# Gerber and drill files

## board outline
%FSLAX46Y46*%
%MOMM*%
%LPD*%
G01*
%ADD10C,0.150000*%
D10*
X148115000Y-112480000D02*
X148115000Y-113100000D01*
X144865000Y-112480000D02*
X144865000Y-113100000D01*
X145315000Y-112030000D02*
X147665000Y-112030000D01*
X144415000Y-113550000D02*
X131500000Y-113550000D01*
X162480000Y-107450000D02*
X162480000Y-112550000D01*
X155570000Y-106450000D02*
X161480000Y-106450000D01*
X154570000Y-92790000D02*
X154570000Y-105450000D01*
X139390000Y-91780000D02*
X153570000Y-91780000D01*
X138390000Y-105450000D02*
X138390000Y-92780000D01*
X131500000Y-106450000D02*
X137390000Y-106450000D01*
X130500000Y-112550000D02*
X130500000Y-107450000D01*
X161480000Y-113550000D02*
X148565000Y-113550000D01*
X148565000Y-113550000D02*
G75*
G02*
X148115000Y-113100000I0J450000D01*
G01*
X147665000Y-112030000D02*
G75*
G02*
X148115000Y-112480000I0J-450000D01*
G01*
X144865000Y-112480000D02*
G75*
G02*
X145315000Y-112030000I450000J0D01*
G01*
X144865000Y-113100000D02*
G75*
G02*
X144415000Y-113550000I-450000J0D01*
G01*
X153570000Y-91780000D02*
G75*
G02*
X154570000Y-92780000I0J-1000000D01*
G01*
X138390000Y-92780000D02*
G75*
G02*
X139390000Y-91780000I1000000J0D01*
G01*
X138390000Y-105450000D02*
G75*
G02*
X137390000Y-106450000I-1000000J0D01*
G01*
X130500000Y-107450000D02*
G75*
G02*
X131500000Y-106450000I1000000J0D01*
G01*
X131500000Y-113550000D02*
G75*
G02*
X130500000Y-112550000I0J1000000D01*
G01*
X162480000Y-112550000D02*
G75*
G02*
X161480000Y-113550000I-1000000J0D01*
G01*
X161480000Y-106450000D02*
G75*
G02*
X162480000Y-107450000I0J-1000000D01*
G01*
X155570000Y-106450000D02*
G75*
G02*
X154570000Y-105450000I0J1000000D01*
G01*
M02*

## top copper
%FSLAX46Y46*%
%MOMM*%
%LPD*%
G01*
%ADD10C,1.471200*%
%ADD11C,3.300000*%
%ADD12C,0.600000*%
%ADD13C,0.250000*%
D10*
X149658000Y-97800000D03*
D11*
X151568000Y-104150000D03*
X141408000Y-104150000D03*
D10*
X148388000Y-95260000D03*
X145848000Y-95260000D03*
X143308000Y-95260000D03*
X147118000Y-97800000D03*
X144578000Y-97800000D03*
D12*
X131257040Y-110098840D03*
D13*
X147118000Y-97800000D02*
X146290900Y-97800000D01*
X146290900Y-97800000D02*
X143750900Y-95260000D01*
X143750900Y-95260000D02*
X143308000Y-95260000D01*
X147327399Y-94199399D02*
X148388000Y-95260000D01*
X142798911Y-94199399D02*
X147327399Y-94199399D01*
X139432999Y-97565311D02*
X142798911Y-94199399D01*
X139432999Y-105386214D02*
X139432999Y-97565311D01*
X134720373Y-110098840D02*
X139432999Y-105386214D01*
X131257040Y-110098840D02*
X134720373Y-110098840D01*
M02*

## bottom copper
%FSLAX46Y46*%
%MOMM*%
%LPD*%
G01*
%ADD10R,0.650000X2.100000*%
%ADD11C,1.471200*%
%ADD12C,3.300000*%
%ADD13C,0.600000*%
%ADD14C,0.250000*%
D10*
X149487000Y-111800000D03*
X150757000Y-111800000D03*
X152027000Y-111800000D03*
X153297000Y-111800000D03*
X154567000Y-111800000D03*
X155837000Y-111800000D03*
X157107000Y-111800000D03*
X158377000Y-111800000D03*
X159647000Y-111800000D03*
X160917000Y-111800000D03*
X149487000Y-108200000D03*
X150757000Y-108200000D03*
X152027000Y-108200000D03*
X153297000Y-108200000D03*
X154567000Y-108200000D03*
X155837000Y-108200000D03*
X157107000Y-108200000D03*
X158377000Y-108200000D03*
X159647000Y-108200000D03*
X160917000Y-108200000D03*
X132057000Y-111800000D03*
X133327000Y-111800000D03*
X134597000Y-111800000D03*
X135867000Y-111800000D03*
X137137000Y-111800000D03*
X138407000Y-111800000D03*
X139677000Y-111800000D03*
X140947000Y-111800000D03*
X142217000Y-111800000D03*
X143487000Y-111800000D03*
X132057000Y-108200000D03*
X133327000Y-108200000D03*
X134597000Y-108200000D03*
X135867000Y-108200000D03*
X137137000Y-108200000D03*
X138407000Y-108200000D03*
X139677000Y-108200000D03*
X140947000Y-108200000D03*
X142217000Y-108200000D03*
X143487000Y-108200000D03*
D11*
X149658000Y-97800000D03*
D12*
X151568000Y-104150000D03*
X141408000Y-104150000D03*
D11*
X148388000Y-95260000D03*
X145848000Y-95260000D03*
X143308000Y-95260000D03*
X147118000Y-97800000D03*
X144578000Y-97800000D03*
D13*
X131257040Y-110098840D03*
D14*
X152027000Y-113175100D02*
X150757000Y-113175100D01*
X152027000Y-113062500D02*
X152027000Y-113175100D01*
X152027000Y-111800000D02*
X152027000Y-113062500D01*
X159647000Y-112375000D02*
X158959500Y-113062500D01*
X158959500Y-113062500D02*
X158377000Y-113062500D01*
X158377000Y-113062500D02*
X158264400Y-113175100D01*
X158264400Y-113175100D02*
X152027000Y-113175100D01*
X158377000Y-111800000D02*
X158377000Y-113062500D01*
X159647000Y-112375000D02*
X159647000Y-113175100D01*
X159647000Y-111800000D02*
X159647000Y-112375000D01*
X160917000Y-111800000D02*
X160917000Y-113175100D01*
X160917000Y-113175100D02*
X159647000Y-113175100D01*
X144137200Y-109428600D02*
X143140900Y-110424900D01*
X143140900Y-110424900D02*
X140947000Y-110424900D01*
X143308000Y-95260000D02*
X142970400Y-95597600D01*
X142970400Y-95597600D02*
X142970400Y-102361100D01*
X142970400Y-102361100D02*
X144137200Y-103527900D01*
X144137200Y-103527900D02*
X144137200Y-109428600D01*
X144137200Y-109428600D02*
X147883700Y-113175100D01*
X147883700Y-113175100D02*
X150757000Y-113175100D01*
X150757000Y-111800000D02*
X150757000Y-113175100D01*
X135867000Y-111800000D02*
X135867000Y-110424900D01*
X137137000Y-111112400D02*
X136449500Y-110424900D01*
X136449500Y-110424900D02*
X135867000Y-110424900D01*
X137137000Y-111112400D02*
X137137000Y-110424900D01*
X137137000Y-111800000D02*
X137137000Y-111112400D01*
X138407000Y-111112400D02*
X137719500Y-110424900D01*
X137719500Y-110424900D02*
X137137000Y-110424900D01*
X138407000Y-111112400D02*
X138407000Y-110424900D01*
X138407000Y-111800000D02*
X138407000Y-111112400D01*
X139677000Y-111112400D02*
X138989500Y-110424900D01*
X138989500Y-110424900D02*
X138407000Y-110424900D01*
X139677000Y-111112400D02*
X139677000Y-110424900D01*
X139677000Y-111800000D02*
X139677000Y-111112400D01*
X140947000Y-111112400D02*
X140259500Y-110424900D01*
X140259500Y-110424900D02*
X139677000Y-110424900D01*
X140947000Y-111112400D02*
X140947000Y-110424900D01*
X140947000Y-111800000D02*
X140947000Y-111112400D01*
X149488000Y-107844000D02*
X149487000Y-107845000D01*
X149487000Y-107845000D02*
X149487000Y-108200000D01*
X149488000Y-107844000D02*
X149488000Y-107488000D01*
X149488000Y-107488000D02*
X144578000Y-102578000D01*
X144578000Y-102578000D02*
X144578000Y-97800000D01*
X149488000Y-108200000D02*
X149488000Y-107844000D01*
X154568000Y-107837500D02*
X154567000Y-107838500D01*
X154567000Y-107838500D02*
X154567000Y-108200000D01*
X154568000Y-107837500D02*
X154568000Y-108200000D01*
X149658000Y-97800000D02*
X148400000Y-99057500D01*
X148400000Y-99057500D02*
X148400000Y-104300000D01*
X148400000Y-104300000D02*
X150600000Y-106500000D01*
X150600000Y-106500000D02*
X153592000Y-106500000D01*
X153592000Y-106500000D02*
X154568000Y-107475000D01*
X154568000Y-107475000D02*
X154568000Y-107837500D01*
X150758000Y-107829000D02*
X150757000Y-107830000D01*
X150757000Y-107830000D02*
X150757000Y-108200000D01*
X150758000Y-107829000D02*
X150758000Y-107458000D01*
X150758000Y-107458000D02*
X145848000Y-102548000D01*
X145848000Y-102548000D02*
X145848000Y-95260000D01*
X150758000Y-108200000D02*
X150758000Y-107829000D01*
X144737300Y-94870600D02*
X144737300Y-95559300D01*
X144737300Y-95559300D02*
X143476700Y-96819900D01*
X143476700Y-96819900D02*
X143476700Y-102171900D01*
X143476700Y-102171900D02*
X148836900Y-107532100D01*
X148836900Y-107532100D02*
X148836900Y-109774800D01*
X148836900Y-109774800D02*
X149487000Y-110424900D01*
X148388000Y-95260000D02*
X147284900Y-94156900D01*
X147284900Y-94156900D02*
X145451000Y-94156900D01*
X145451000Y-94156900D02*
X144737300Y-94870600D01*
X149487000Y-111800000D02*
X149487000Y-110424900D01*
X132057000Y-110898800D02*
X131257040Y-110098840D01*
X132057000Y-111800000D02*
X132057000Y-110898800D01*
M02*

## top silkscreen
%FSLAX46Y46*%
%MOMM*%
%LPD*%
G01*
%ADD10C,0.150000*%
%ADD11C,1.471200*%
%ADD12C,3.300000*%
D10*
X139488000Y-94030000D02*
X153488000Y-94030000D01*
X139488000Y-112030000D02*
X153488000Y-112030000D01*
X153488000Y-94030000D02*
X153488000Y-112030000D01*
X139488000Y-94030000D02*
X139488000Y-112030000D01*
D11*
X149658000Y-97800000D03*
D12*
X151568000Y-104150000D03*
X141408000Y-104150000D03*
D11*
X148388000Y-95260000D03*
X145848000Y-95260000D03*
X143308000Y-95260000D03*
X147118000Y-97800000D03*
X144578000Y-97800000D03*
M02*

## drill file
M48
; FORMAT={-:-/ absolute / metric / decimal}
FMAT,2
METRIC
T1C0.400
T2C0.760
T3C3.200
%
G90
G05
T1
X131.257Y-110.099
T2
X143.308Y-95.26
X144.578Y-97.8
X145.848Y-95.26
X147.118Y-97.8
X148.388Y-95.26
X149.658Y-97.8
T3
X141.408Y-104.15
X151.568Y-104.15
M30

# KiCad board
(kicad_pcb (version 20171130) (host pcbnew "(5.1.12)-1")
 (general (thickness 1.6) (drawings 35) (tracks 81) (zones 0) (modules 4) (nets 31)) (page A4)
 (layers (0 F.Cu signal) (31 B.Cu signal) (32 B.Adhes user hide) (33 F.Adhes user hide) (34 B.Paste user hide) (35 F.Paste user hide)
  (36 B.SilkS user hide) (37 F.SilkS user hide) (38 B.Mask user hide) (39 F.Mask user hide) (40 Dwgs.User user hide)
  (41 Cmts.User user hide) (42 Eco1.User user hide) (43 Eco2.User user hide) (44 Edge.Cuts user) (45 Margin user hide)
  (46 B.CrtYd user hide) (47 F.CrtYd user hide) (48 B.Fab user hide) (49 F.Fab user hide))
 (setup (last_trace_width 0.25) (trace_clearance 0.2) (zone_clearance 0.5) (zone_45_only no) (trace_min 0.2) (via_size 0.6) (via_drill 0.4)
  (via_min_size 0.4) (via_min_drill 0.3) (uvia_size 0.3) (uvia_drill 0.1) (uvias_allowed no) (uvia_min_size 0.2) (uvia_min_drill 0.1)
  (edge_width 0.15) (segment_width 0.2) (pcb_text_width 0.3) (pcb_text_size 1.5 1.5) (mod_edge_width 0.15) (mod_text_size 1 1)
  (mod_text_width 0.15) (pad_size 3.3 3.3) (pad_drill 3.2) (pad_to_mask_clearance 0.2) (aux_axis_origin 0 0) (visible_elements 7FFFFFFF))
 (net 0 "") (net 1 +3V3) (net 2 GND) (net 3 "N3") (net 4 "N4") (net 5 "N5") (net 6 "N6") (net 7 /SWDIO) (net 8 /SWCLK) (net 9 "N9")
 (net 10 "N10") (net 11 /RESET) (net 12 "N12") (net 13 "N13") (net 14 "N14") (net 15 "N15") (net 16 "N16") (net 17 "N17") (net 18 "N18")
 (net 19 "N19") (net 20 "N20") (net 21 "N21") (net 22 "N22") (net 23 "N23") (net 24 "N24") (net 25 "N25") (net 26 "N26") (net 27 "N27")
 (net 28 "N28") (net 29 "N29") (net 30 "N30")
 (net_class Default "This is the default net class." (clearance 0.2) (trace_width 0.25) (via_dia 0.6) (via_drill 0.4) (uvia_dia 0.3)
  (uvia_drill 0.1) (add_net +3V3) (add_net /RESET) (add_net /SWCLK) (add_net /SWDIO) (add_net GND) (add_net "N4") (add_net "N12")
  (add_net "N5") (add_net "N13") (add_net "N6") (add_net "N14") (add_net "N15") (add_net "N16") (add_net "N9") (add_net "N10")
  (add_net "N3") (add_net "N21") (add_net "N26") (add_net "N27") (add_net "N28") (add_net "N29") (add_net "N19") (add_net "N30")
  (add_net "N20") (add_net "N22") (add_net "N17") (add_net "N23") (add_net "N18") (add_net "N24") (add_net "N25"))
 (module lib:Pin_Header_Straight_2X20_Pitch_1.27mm (layer B.Cu) (at 155.202 110)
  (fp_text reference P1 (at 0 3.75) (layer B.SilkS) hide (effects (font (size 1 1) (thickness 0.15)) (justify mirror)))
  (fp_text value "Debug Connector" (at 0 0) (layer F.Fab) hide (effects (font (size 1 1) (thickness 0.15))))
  (pad 2 smd rect (at -5.715 1.8) (size 0.65 2.1) (layers B.Cu B.Paste B.Mask) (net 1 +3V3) (solder_mask_margin 0.1))
  (pad 4 smd rect (at -4.445 1.8) (size 0.65 2.1) (layers B.Cu B.Paste B.Mask) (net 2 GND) (solder_mask_margin 0.1))
  (pad 6 smd rect (at -3.175 1.8) (size 0.65 2.1) (layers B.Cu B.Paste B.Mask) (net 2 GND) (solder_mask_margin 0.1))
  (pad 8 smd rect (at -1.905 1.8) (size 0.65 2.1) (layers B.Cu B.Paste B.Mask) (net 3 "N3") (solder_mask_margin 0.1))
  (pad 10 smd rect (at -0.635 1.8) (size 0.65 2.1) (layers B.Cu B.Paste B.Mask) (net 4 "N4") (solder_mask_margin 0.1))
  (pad 12 smd rect (at 0.635 1.8) (size 0.65 2.1) (layers B.Cu B.Paste B.Mask) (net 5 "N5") (solder_mask_margin 0.1))
  (pad 14 smd rect (at 1.905 1.8) (size 0.65 2.1) (layers B.Cu B.Paste B.Mask) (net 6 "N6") (solder_mask_margin 0.1))
  (pad 16 smd rect (at 3.175 1.8) (size 0.65 2.1) (layers B.Cu B.Paste B.Mask) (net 2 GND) (solder_mask_margin 0.1))
  (pad 18 smd rect (at 4.445 1.8) (size 0.65 2.1) (layers B.Cu B.Paste B.Mask) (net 2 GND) (solder_mask_margin 0.1))
  (pad 20 smd rect (at 5.715 1.8) (size 0.65 2.1) (layers B.Cu B.Paste B.Mask) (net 2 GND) (solder_mask_margin 0.1))
  (pad 1 smd rect (at -5.715 -1.8) (size 0.65 2.1) (layers B.Cu B.Paste B.Mask) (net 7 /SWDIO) (solder_mask_margin 0.1))
  (pad 3 smd rect (at -4.445 -1.8) (size 0.65 2.1) (layers B.Cu B.Paste B.Mask) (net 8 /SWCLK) (solder_mask_margin 0.1))
  (pad 5 smd rect (at -3.175 -1.8) (size 0.65 2.1) (layers B.Cu B.Paste B.Mask) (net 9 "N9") (solder_mask_margin 0.1))
  (pad 7 smd rect (at -1.905 -1.8) (size 0.65 2.1) (layers B.Cu B.Paste B.Mask) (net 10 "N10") (solder_mask_margin 0.1))
  (pad 9 smd rect (at -0.635 -1.8) (size 0.65 2.1) (layers B.Cu B.Paste B.Mask) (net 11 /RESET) (solder_mask_margin 0.1))
  (pad 11 smd rect (at 0.635 -1.8) (size 0.65 2.1) (layers B.Cu B.Paste B.Mask) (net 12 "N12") (solder_mask_margin 0.1))
  (pad 13 smd rect (at 1.905 -1.8) (size 0.65 2.1) (layers B.Cu B.Paste B.Mask) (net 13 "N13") (solder_mask_margin 0.1))
  (pad 15 smd rect (at 3.175 -1.8) (size 0.65 2.1) (layers B.Cu B.Paste B.Mask) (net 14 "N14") (solder_mask_margin 0.1))
  (pad 17 smd rect (at 4.445 -1.8) (size 0.65 2.1) (layers B.Cu B.Paste B.Mask) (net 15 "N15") (solder_mask_margin 0.1))
  (pad 19 smd rect (at 5.715 -1.8) (size 0.65 2.1) (layers B.Cu B.Paste B.Mask) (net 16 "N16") (solder_mask_margin 0.1)))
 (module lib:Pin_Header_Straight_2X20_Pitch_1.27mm (layer B.Cu) (at 137.772 110)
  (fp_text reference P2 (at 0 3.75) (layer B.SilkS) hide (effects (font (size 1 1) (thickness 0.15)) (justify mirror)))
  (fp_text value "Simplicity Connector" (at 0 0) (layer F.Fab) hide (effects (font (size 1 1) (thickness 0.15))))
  (pad 2 smd rect (at -5.715 1.8) (size 0.65 2.1) (layers B.Cu B.Paste B.Mask) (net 1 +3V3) (solder_mask_margin 0.1))
  (pad 4 smd rect (at -4.445 1.8) (size 0.65 2.1) (layers B.Cu B.Paste B.Mask) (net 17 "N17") (solder_mask_margin 0.1))
  (pad 6 smd rect (at -3.175 1.8) (size 0.65 2.1) (layers B.Cu B.Paste B.Mask) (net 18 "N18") (solder_mask_margin 0.1))
  (pad 8 smd rect (at -1.905 1.8) (size 0.65 2.1) (layers B.Cu B.Paste B.Mask) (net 2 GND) (solder_mask_margin 0.1))
  (pad 10 smd rect (at -0.635 1.8) (size 0.65 2.1) (layers B.Cu B.Paste B.Mask) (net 2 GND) (solder_mask_margin 0.1))
  (pad 12 smd rect (at 0.635 1.8) (size 0.65 2.1) (layers B.Cu B.Paste B.Mask) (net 2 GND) (solder_mask_margin 0.1))
  (pad 14 smd rect (at 1.905 1.8) (size 0.65 2.1) (layers B.Cu B.Paste B.Mask) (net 2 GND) (solder_mask_margin 0.1))
  (pad 16 smd rect (at 3.175 1.8) (size 0.65 2.1) (layers B.Cu B.Paste B.Mask) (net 2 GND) (solder_mask_margin 0.1))
  (pad 18 smd rect (at 4.445 1.8) (size 0.65 2.1) (layers B.Cu B.Paste B.Mask) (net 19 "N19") (solder_mask_margin 0.1))
  (pad 20 smd rect (at 5.715 1.8) (size 0.65 2.1) (layers B.Cu B.Paste B.Mask) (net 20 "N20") (solder_mask_margin 0.1))
  (pad 1 smd rect (at -5.715 -1.8) (size 0.65 2.1) (layers B.Cu B.Paste B.Mask) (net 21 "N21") (solder_mask_margin 0.1))
  (pad 3 smd rect (at -4.445 -1.8) (size 0.65 2.1) (layers B.Cu B.Paste B.Mask) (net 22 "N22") (solder_mask_margin 0.1))
  (pad 5 smd rect (at -3.175 -1.8) (size 0.65 2.1) (layers B.Cu B.Paste B.Mask) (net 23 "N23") (solder_mask_margin 0.1))
  (pad 7 smd rect (at -1.905 -1.8) (size 0.65 2.1) (layers B.Cu B.Paste B.Mask) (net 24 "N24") (solder_mask_margin 0.1))
  (pad 9 smd rect (at -0.635 -1.8) (size 0.65 2.1) (layers B.Cu B.Paste B.Mask) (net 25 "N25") (solder_mask_margin 0.1))
  (pad 11 smd rect (at 0.635 -1.8) (size 0.65 2.1) (layers B.Cu B.Paste B.Mask) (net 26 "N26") (solder_mask_margin 0.1))
  (pad 13 smd rect (at 1.905 -1.8) (size 0.65 2.1) (layers B.Cu B.Paste B.Mask) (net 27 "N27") (solder_mask_margin 0.1))
  (pad 15 smd rect (at 3.175 -1.8) (size 0.65 2.1) (layers B.Cu B.Paste B.Mask) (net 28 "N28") (solder_mask_margin 0.1))
  (pad 17 smd rect (at 4.445 -1.8) (size 0.65 2.1) (layers B.Cu B.Paste B.Mask) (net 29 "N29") (solder_mask_margin 0.1))
  (pad 19 smd rect (at 5.715 -1.8) (size 0.65 2.1) (layers B.Cu B.Paste B.Mask) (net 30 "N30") (solder_mask_margin 0.1)))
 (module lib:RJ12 (layer F.Cu) (at 146.488 104.15)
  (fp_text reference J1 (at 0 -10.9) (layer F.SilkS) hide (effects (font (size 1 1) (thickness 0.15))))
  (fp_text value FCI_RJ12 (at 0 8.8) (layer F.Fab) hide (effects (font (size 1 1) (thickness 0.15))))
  (fp_line (start -7 -10.12) (end 7 -10.12) (layer F.SilkS) (width 0.15))
  (fp_line (start -7 7.88) (end 7 7.88) (layer F.SilkS) (width 0.15))
  (fp_line (start 7 -10.12) (end 7 7.88) (layer F.SilkS) (width 0.15))
  (fp_line (start -7 -10.12) (end -7 7.88) (layer F.SilkS) (width 0.15))
  (pad 6 thru_hole circle (at 3.17 -6.35) (size 1.4712 1.4712) (drill 0.76) (layers *.Cu *.Mask F.SilkS) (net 11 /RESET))
  (pad "" np_thru_hole circle (at 5.08 0) (size 3.3 3.3) (drill 3.2) (layers *.Cu *.Mask F.SilkS))
  (pad "" np_thru_hole circle (at -5.08 0) (size 3.3 3.3) (drill 3.2) (layers *.Cu *.Mask F.SilkS))
  (pad 5 thru_hole circle (at 1.9 -8.89) (size 1.4712 1.4712) (drill 0.76) (layers *.Cu *.Mask F.SilkS) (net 1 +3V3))
  (pad 3 thru_hole circle (at -0.64 -8.89) (size 1.4712 1.4712) (drill 0.76) (layers *.Cu *.Mask F.SilkS) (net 8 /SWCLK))
  (pad 1 thru_hole circle (at -3.18 -8.89) (size 1.4712 1.4712) (drill 0.76) (layers *.Cu *.Mask F.SilkS) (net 2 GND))
  (pad 4 thru_hole circle (at 0.63 -6.35) (size 1.4712 1.4712) (drill 0.76) (layers *.Cu *.Mask F.SilkS) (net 2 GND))
  (pad 2 thru_hole circle (at -1.91 -6.35) (size 1.4712 1.4712) (drill 0.76) (layers *.Cu *.Mask F.SilkS) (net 7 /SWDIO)))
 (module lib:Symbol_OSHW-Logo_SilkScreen (layer B.Cu) (at 146.488 102 180)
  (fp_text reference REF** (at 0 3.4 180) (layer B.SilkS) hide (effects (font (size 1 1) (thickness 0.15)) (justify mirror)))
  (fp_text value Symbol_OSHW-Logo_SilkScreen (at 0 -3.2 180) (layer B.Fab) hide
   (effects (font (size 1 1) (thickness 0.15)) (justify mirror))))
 (gr_line (start 148.115 112.48) (end 148.115 113.1) (layer Edge.Cuts) (width 0.15))
 (gr_line (start 144.865 112.48) (end 144.865 113.1) (layer Edge.Cuts) (width 0.15))
 (gr_line (start 145.315 112.03) (end 147.665 112.03) (layer Edge.Cuts) (width 0.15))
 (gr_line (start 144.415 113.55) (end 131.5 113.55) (layer Edge.Cuts) (width 0.15))
 (gr_line (start 162.48 107.45) (end 162.48 112.55) (layer Edge.Cuts) (width 0.15))
 (gr_line (start 155.57 106.45) (end 161.48 106.45) (layer Edge.Cuts) (width 0.15))
 (gr_line (start 154.57 92.79) (end 154.57 105.45) (layer Edge.Cuts) (width 0.15))
 (gr_line (start 139.39 91.78) (end 153.57 91.78) (layer Edge.Cuts) (width 0.15))
 (gr_line (start 138.39 105.45) (end 138.39 92.78) (layer Edge.Cuts) (width 0.15))
 (gr_line (start 131.5 106.45) (end 137.39 106.45) (layer Edge.Cuts) (width 0.15))
 (gr_line (start 130.5 112.55) (end 130.5 107.45) (layer Edge.Cuts) (width 0.15))
 (gr_line (start 161.48 113.55) (end 148.565 113.55) (layer Edge.Cuts) (width 0.15))
 (gr_arc (start 148.565 113.1) (end 148.565 113.55) (angle 90) (layer Edge.Cuts) (width 0.15))
 (gr_arc (start 147.665 112.48) (end 147.665 112.03) (angle 90) (layer Edge.Cuts) (width 0.15))
 (gr_arc (start 145.315 112.48) (end 144.865 112.48) (angle 90) (layer Edge.Cuts) (width 0.15))
 (gr_arc (start 144.415 113.1) (end 144.865 113.1) (angle 90) (layer Edge.Cuts) (width 0.15))
 (gr_arc (start 153.57 92.78) (end 153.57 91.78) (angle 90) (layer Edge.Cuts) (width 0.15))
 (gr_arc (start 139.39 92.78) (end 138.39 92.78) (angle 90) (layer Edge.Cuts) (width 0.15))
 (gr_arc (start 137.39 105.45) (end 138.39 105.45) (angle 90) (layer Edge.Cuts) (width 0.15))
 (gr_arc (start 131.5 107.45) (end 130.5 107.45) (angle 90) (layer Edge.Cuts) (width 0.15))
 (gr_arc (start 131.5 112.55) (end 131.5 113.55) (angle 90) (layer Edge.Cuts) (width 0.15))
 (gr_arc (start 161.48 112.55) (end 162.48 112.55) (angle 90) (layer Edge.Cuts) (width 0.15))
 (gr_arc (start 161.48 107.45) (end 161.48 106.45) (angle 90) (layer Edge.Cuts) (width 0.15))
 (gr_arc (start 155.57 105.45) (end 155.57 106.45) (angle 90) (layer Edge.Cuts) (width 0.15))
 (via (at 131.25704 110.09884) (size 0.6) (drill 0.4) (layers F.Cu B.Cu) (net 1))
 (segment (start 152.027 113.1751) (end 150.757 113.1751) (width 0.25) (layer B.Cu) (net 2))
 (segment (start 152.027 113.0625) (end 152.027 113.1751) (width 0.25) (layer B.Cu) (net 2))
 (segment (start 152.027 111.8) (end 152.027 113.0625) (width 0.25) (layer B.Cu) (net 2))
 (segment (start 159.647 112.375) (end 158.9595 113.0625) (width 0.25) (layer B.Cu) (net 2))
 (segment (start 158.9595 113.0625) (end 158.377 113.0625) (width 0.25) (layer B.Cu) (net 2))
 (segment (start 158.377 113.0625) (end 158.2644 113.1751) (width 0.25) (layer B.Cu) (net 2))
 (segment (start 158.2644 113.1751) (end 152.027 113.1751) (width 0.25) (layer B.Cu) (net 2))
 (segment (start 158.377 111.8) (end 158.377 113.0625) (width 0.25) (layer B.Cu) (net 2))
 (segment (start 159.647 112.375) (end 159.647 113.1751) (width 0.25) (layer B.Cu) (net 2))
 (segment (start 159.647 111.8) (end 159.647 112.375) (width 0.25) (layer B.Cu) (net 2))
 (segment (start 160.917 111.8) (end 160.917 113.1751) (width 0.25) (layer B.Cu) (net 2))
 (segment (start 160.917 113.1751) (end 159.647 113.1751) (width 0.25) (layer B.Cu) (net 2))
 (segment (start 144.1372 109.4286) (end 143.1409 110.4249) (width 0.25) (layer B.Cu) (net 2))
 (segment (start 143.1409 110.4249) (end 140.947 110.4249) (width 0.25) (layer B.Cu) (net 2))
 (segment (start 143.308 95.26) (end 142.9704 95.5976) (width 0.25) (layer B.Cu) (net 2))
 (segment (start 142.9704 95.5976) (end 142.9704 102.3611) (width 0.25) (layer B.Cu) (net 2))
 (segment (start 142.9704 102.3611) (end 144.1372 103.5279) (width 0.25) (layer B.Cu) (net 2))
 (segment (start 144.1372 103.5279) (end 144.1372 109.4286) (width 0.25) (layer B.Cu) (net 2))
 (segment (start 144.1372 109.4286) (end 147.8837 113.1751) (width 0.25) (layer B.Cu) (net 2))
 (segment (start 147.8837 113.1751) (end 150.757 113.1751) (width 0.25) (layer B.Cu) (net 2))
 (segment (start 150.757 111.8) (end 150.757 113.1751) (width 0.25) (layer B.Cu) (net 2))
 (segment (start 135.867 111.8) (end 135.867 110.4249) (width 0.25) (layer B.Cu) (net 2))
 (segment (start 137.137 111.1124) (end 136.4495 110.4249) (width 0.25) (layer B.Cu) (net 2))
 (segment (start 136.4495 110.4249) (end 135.867 110.4249) (width 0.25) (layer B.Cu) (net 2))
 (segment (start 137.137 111.1124) (end 137.137 110.4249) (width 0.25) (layer B.Cu) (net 2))
 (segment (start 137.137 111.8) (end 137.137 111.1124) (width 0.25) (layer B.Cu) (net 2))
 (segment (start 138.407 111.1124) (end 137.7195 110.4249) (width 0.25) (layer B.Cu) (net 2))
 (segment (start 137.7195 110.4249) (end 137.137 110.4249) (width 0.25) (layer B.Cu) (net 2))
 (segment (start 138.407 111.1124) (end 138.407 110.4249) (width 0.25) (layer B.Cu) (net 2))
 (segment (start 138.407 111.8) (end 138.407 111.1124) (width 0.25) (layer B.Cu) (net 2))
 (segment (start 139.677 111.1124) (end 138.9895 110.4249) (width 0.25) (layer B.Cu) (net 2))
 (segment (start 138.9895 110.4249) (end 138.407 110.4249) (width 0.25) (layer B.Cu) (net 2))
 (segment (start 139.677 111.1124) (end 139.677 110.4249) (width 0.25) (layer B.Cu) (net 2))
 (segment (start 139.677 111.8) (end 139.677 111.1124) (width 0.25) (layer B.Cu) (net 2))
 (segment (start 140.947 111.1124) (end 140.2595 110.4249) (width 0.25) (layer B.Cu) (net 2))
 (segment (start 140.2595 110.4249) (end 139.677 110.4249) (width 0.25) (layer B.Cu) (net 2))
 (segment (start 140.947 111.1124) (end 140.947 110.4249) (width 0.25) (layer B.Cu) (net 2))
 (segment (start 140.947 111.8) (end 140.947 111.1124) (width 0.25) (layer B.Cu) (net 2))
 (segment (start 147.118 97.8) (end 146.2909 97.8) (width 0.25) (layer F.Cu) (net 2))
 (segment (start 146.2909 97.8) (end 143.7509 95.26) (width 0.25) (layer F.Cu) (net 2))
 (segment (start 143.7509 95.26) (end 143.308 95.26) (width 0.25) (layer F.Cu) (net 2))
 (segment (start 149.488 107.844) (end 149.487 107.845) (width 0.25) (layer B.Cu) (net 7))
 (segment (start 149.487 107.845) (end 149.487 108.2) (width 0.25) (layer B.Cu) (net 7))
 (segment (start 149.488 107.844) (end 149.488 107.488) (width 0.25) (layer B.Cu) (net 7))
 (segment (start 149.488 107.488) (end 144.578 102.578) (width 0.25) (layer B.Cu) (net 7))
 (segment (start 144.578 102.578) (end 144.578 97.8) (width 0.25) (layer B.Cu) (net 7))
 (segment (start 149.488 108.2) (end 149.488 107.844) (width 0.25) (layer B.Cu) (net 7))
 (segment (start 154.568 107.8375) (end 154.567 107.8385) (width 0.25) (layer B.Cu) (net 11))
 (segment (start 154.567 107.8385) (end 154.567 108.2) (width 0.25) (layer B.Cu) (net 11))
 (segment (start 154.568 107.8375) (end 154.568 108.2) (width 0.25) (layer B.Cu) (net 11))
 (segment (start 149.658 97.8) (end 148.4 99.0575) (width 0.25) (layer B.Cu) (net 11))
 (segment (start 148.4 99.0575) (end 148.4 104.3) (width 0.25) (layer B.Cu) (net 11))
 (segment (start 148.4 104.3) (end 150.6 106.5) (width 0.25) (layer B.Cu) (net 11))
 (segment (start 150.6 106.5) (end 153.592 106.5) (width 0.25) (layer B.Cu) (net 11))
 (segment (start 153.592 106.5) (end 154.568 107.475) (width 0.25) (layer B.Cu) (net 11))
 (segment (start 154.568 107.475) (end 154.568 107.8375) (width 0.25) (layer B.Cu) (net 11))
 (segment (start 150.758 107.829) (end 150.757 107.83) (width 0.25) (layer B.Cu) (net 8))
 (segment (start 150.757 107.83) (end 150.757 108.2) (width 0.25) (layer B.Cu) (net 8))
 (segment (start 150.758 107.829) (end 150.758 107.458) (width 0.25) (layer B.Cu) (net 8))
 (segment (start 150.758 107.458) (end 145.848 102.548) (width 0.25) (layer B.Cu) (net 8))
 (segment (start 145.848 102.548) (end 145.848 95.26) (width 0.25) (layer B.Cu) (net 8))
 (segment (start 150.758 108.2) (end 150.758 107.829) (width 0.25) (layer B.Cu) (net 8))
 (segment (start 144.7373 94.8706) (end 144.7373 95.5593) (width 0.25) (layer B.Cu) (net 1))
 (segment (start 144.7373 95.5593) (end 143.4767 96.8199) (width 0.25) (layer B.Cu) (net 1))
 (segment (start 143.4767 96.8199) (end 143.4767 102.1719) (width 0.25) (layer B.Cu) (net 1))
 (segment (start 143.4767 102.1719) (end 148.8369 107.5321) (width 0.25) (layer B.Cu) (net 1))
 (segment (start 148.8369 107.5321) (end 148.8369 109.7748) (width 0.25) (layer B.Cu) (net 1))
 (segment (start 148.8369 109.7748) (end 149.487 110.4249) (width 0.25) (layer B.Cu) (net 1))
 (segment (start 148.388 95.26) (end 147.2849 94.1569) (width 0.25) (layer B.Cu) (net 1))
 (segment (start 147.2849 94.1569) (end 145.451 94.1569) (width 0.25) (layer B.Cu) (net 1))
 (segment (start 145.451 94.1569) (end 144.7373 94.8706) (width 0.25) (layer B.Cu) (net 1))
 (segment (start 149.487 111.8) (end 149.487 110.4249) (width 0.25) (layer B.Cu) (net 1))
 (segment (start 132.057 110.8988) (end 131.25704 110.09884) (width 0.25) (layer B.Cu) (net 1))
 (segment (start 132.057 111.8) (end 132.057 110.8988) (width 0.25) (layer B.Cu) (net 1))
 (segment (start 147.327399 94.199399) (end 148.388 95.26) (width 0.25) (layer F.Cu) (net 1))
 (segment (start 142.798911 94.199399) (end 147.327399 94.199399) (width 0.25) (layer F.Cu) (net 1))
 (segment (start 139.432999 97.565311) (end 142.798911 94.199399) (width 0.25) (layer F.Cu) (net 1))
 (segment (start 139.432999 105.386214) (end 139.432999 97.565311) (width 0.25) (layer F.Cu) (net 1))
 (segment (start 134.720373 110.09884) (end 139.432999 105.386214) (width 0.25) (layer F.Cu) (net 1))
 (segment (start 131.25704 110.09884) (end 134.720373 110.09884) (width 0.25) (layer F.Cu) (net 1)))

